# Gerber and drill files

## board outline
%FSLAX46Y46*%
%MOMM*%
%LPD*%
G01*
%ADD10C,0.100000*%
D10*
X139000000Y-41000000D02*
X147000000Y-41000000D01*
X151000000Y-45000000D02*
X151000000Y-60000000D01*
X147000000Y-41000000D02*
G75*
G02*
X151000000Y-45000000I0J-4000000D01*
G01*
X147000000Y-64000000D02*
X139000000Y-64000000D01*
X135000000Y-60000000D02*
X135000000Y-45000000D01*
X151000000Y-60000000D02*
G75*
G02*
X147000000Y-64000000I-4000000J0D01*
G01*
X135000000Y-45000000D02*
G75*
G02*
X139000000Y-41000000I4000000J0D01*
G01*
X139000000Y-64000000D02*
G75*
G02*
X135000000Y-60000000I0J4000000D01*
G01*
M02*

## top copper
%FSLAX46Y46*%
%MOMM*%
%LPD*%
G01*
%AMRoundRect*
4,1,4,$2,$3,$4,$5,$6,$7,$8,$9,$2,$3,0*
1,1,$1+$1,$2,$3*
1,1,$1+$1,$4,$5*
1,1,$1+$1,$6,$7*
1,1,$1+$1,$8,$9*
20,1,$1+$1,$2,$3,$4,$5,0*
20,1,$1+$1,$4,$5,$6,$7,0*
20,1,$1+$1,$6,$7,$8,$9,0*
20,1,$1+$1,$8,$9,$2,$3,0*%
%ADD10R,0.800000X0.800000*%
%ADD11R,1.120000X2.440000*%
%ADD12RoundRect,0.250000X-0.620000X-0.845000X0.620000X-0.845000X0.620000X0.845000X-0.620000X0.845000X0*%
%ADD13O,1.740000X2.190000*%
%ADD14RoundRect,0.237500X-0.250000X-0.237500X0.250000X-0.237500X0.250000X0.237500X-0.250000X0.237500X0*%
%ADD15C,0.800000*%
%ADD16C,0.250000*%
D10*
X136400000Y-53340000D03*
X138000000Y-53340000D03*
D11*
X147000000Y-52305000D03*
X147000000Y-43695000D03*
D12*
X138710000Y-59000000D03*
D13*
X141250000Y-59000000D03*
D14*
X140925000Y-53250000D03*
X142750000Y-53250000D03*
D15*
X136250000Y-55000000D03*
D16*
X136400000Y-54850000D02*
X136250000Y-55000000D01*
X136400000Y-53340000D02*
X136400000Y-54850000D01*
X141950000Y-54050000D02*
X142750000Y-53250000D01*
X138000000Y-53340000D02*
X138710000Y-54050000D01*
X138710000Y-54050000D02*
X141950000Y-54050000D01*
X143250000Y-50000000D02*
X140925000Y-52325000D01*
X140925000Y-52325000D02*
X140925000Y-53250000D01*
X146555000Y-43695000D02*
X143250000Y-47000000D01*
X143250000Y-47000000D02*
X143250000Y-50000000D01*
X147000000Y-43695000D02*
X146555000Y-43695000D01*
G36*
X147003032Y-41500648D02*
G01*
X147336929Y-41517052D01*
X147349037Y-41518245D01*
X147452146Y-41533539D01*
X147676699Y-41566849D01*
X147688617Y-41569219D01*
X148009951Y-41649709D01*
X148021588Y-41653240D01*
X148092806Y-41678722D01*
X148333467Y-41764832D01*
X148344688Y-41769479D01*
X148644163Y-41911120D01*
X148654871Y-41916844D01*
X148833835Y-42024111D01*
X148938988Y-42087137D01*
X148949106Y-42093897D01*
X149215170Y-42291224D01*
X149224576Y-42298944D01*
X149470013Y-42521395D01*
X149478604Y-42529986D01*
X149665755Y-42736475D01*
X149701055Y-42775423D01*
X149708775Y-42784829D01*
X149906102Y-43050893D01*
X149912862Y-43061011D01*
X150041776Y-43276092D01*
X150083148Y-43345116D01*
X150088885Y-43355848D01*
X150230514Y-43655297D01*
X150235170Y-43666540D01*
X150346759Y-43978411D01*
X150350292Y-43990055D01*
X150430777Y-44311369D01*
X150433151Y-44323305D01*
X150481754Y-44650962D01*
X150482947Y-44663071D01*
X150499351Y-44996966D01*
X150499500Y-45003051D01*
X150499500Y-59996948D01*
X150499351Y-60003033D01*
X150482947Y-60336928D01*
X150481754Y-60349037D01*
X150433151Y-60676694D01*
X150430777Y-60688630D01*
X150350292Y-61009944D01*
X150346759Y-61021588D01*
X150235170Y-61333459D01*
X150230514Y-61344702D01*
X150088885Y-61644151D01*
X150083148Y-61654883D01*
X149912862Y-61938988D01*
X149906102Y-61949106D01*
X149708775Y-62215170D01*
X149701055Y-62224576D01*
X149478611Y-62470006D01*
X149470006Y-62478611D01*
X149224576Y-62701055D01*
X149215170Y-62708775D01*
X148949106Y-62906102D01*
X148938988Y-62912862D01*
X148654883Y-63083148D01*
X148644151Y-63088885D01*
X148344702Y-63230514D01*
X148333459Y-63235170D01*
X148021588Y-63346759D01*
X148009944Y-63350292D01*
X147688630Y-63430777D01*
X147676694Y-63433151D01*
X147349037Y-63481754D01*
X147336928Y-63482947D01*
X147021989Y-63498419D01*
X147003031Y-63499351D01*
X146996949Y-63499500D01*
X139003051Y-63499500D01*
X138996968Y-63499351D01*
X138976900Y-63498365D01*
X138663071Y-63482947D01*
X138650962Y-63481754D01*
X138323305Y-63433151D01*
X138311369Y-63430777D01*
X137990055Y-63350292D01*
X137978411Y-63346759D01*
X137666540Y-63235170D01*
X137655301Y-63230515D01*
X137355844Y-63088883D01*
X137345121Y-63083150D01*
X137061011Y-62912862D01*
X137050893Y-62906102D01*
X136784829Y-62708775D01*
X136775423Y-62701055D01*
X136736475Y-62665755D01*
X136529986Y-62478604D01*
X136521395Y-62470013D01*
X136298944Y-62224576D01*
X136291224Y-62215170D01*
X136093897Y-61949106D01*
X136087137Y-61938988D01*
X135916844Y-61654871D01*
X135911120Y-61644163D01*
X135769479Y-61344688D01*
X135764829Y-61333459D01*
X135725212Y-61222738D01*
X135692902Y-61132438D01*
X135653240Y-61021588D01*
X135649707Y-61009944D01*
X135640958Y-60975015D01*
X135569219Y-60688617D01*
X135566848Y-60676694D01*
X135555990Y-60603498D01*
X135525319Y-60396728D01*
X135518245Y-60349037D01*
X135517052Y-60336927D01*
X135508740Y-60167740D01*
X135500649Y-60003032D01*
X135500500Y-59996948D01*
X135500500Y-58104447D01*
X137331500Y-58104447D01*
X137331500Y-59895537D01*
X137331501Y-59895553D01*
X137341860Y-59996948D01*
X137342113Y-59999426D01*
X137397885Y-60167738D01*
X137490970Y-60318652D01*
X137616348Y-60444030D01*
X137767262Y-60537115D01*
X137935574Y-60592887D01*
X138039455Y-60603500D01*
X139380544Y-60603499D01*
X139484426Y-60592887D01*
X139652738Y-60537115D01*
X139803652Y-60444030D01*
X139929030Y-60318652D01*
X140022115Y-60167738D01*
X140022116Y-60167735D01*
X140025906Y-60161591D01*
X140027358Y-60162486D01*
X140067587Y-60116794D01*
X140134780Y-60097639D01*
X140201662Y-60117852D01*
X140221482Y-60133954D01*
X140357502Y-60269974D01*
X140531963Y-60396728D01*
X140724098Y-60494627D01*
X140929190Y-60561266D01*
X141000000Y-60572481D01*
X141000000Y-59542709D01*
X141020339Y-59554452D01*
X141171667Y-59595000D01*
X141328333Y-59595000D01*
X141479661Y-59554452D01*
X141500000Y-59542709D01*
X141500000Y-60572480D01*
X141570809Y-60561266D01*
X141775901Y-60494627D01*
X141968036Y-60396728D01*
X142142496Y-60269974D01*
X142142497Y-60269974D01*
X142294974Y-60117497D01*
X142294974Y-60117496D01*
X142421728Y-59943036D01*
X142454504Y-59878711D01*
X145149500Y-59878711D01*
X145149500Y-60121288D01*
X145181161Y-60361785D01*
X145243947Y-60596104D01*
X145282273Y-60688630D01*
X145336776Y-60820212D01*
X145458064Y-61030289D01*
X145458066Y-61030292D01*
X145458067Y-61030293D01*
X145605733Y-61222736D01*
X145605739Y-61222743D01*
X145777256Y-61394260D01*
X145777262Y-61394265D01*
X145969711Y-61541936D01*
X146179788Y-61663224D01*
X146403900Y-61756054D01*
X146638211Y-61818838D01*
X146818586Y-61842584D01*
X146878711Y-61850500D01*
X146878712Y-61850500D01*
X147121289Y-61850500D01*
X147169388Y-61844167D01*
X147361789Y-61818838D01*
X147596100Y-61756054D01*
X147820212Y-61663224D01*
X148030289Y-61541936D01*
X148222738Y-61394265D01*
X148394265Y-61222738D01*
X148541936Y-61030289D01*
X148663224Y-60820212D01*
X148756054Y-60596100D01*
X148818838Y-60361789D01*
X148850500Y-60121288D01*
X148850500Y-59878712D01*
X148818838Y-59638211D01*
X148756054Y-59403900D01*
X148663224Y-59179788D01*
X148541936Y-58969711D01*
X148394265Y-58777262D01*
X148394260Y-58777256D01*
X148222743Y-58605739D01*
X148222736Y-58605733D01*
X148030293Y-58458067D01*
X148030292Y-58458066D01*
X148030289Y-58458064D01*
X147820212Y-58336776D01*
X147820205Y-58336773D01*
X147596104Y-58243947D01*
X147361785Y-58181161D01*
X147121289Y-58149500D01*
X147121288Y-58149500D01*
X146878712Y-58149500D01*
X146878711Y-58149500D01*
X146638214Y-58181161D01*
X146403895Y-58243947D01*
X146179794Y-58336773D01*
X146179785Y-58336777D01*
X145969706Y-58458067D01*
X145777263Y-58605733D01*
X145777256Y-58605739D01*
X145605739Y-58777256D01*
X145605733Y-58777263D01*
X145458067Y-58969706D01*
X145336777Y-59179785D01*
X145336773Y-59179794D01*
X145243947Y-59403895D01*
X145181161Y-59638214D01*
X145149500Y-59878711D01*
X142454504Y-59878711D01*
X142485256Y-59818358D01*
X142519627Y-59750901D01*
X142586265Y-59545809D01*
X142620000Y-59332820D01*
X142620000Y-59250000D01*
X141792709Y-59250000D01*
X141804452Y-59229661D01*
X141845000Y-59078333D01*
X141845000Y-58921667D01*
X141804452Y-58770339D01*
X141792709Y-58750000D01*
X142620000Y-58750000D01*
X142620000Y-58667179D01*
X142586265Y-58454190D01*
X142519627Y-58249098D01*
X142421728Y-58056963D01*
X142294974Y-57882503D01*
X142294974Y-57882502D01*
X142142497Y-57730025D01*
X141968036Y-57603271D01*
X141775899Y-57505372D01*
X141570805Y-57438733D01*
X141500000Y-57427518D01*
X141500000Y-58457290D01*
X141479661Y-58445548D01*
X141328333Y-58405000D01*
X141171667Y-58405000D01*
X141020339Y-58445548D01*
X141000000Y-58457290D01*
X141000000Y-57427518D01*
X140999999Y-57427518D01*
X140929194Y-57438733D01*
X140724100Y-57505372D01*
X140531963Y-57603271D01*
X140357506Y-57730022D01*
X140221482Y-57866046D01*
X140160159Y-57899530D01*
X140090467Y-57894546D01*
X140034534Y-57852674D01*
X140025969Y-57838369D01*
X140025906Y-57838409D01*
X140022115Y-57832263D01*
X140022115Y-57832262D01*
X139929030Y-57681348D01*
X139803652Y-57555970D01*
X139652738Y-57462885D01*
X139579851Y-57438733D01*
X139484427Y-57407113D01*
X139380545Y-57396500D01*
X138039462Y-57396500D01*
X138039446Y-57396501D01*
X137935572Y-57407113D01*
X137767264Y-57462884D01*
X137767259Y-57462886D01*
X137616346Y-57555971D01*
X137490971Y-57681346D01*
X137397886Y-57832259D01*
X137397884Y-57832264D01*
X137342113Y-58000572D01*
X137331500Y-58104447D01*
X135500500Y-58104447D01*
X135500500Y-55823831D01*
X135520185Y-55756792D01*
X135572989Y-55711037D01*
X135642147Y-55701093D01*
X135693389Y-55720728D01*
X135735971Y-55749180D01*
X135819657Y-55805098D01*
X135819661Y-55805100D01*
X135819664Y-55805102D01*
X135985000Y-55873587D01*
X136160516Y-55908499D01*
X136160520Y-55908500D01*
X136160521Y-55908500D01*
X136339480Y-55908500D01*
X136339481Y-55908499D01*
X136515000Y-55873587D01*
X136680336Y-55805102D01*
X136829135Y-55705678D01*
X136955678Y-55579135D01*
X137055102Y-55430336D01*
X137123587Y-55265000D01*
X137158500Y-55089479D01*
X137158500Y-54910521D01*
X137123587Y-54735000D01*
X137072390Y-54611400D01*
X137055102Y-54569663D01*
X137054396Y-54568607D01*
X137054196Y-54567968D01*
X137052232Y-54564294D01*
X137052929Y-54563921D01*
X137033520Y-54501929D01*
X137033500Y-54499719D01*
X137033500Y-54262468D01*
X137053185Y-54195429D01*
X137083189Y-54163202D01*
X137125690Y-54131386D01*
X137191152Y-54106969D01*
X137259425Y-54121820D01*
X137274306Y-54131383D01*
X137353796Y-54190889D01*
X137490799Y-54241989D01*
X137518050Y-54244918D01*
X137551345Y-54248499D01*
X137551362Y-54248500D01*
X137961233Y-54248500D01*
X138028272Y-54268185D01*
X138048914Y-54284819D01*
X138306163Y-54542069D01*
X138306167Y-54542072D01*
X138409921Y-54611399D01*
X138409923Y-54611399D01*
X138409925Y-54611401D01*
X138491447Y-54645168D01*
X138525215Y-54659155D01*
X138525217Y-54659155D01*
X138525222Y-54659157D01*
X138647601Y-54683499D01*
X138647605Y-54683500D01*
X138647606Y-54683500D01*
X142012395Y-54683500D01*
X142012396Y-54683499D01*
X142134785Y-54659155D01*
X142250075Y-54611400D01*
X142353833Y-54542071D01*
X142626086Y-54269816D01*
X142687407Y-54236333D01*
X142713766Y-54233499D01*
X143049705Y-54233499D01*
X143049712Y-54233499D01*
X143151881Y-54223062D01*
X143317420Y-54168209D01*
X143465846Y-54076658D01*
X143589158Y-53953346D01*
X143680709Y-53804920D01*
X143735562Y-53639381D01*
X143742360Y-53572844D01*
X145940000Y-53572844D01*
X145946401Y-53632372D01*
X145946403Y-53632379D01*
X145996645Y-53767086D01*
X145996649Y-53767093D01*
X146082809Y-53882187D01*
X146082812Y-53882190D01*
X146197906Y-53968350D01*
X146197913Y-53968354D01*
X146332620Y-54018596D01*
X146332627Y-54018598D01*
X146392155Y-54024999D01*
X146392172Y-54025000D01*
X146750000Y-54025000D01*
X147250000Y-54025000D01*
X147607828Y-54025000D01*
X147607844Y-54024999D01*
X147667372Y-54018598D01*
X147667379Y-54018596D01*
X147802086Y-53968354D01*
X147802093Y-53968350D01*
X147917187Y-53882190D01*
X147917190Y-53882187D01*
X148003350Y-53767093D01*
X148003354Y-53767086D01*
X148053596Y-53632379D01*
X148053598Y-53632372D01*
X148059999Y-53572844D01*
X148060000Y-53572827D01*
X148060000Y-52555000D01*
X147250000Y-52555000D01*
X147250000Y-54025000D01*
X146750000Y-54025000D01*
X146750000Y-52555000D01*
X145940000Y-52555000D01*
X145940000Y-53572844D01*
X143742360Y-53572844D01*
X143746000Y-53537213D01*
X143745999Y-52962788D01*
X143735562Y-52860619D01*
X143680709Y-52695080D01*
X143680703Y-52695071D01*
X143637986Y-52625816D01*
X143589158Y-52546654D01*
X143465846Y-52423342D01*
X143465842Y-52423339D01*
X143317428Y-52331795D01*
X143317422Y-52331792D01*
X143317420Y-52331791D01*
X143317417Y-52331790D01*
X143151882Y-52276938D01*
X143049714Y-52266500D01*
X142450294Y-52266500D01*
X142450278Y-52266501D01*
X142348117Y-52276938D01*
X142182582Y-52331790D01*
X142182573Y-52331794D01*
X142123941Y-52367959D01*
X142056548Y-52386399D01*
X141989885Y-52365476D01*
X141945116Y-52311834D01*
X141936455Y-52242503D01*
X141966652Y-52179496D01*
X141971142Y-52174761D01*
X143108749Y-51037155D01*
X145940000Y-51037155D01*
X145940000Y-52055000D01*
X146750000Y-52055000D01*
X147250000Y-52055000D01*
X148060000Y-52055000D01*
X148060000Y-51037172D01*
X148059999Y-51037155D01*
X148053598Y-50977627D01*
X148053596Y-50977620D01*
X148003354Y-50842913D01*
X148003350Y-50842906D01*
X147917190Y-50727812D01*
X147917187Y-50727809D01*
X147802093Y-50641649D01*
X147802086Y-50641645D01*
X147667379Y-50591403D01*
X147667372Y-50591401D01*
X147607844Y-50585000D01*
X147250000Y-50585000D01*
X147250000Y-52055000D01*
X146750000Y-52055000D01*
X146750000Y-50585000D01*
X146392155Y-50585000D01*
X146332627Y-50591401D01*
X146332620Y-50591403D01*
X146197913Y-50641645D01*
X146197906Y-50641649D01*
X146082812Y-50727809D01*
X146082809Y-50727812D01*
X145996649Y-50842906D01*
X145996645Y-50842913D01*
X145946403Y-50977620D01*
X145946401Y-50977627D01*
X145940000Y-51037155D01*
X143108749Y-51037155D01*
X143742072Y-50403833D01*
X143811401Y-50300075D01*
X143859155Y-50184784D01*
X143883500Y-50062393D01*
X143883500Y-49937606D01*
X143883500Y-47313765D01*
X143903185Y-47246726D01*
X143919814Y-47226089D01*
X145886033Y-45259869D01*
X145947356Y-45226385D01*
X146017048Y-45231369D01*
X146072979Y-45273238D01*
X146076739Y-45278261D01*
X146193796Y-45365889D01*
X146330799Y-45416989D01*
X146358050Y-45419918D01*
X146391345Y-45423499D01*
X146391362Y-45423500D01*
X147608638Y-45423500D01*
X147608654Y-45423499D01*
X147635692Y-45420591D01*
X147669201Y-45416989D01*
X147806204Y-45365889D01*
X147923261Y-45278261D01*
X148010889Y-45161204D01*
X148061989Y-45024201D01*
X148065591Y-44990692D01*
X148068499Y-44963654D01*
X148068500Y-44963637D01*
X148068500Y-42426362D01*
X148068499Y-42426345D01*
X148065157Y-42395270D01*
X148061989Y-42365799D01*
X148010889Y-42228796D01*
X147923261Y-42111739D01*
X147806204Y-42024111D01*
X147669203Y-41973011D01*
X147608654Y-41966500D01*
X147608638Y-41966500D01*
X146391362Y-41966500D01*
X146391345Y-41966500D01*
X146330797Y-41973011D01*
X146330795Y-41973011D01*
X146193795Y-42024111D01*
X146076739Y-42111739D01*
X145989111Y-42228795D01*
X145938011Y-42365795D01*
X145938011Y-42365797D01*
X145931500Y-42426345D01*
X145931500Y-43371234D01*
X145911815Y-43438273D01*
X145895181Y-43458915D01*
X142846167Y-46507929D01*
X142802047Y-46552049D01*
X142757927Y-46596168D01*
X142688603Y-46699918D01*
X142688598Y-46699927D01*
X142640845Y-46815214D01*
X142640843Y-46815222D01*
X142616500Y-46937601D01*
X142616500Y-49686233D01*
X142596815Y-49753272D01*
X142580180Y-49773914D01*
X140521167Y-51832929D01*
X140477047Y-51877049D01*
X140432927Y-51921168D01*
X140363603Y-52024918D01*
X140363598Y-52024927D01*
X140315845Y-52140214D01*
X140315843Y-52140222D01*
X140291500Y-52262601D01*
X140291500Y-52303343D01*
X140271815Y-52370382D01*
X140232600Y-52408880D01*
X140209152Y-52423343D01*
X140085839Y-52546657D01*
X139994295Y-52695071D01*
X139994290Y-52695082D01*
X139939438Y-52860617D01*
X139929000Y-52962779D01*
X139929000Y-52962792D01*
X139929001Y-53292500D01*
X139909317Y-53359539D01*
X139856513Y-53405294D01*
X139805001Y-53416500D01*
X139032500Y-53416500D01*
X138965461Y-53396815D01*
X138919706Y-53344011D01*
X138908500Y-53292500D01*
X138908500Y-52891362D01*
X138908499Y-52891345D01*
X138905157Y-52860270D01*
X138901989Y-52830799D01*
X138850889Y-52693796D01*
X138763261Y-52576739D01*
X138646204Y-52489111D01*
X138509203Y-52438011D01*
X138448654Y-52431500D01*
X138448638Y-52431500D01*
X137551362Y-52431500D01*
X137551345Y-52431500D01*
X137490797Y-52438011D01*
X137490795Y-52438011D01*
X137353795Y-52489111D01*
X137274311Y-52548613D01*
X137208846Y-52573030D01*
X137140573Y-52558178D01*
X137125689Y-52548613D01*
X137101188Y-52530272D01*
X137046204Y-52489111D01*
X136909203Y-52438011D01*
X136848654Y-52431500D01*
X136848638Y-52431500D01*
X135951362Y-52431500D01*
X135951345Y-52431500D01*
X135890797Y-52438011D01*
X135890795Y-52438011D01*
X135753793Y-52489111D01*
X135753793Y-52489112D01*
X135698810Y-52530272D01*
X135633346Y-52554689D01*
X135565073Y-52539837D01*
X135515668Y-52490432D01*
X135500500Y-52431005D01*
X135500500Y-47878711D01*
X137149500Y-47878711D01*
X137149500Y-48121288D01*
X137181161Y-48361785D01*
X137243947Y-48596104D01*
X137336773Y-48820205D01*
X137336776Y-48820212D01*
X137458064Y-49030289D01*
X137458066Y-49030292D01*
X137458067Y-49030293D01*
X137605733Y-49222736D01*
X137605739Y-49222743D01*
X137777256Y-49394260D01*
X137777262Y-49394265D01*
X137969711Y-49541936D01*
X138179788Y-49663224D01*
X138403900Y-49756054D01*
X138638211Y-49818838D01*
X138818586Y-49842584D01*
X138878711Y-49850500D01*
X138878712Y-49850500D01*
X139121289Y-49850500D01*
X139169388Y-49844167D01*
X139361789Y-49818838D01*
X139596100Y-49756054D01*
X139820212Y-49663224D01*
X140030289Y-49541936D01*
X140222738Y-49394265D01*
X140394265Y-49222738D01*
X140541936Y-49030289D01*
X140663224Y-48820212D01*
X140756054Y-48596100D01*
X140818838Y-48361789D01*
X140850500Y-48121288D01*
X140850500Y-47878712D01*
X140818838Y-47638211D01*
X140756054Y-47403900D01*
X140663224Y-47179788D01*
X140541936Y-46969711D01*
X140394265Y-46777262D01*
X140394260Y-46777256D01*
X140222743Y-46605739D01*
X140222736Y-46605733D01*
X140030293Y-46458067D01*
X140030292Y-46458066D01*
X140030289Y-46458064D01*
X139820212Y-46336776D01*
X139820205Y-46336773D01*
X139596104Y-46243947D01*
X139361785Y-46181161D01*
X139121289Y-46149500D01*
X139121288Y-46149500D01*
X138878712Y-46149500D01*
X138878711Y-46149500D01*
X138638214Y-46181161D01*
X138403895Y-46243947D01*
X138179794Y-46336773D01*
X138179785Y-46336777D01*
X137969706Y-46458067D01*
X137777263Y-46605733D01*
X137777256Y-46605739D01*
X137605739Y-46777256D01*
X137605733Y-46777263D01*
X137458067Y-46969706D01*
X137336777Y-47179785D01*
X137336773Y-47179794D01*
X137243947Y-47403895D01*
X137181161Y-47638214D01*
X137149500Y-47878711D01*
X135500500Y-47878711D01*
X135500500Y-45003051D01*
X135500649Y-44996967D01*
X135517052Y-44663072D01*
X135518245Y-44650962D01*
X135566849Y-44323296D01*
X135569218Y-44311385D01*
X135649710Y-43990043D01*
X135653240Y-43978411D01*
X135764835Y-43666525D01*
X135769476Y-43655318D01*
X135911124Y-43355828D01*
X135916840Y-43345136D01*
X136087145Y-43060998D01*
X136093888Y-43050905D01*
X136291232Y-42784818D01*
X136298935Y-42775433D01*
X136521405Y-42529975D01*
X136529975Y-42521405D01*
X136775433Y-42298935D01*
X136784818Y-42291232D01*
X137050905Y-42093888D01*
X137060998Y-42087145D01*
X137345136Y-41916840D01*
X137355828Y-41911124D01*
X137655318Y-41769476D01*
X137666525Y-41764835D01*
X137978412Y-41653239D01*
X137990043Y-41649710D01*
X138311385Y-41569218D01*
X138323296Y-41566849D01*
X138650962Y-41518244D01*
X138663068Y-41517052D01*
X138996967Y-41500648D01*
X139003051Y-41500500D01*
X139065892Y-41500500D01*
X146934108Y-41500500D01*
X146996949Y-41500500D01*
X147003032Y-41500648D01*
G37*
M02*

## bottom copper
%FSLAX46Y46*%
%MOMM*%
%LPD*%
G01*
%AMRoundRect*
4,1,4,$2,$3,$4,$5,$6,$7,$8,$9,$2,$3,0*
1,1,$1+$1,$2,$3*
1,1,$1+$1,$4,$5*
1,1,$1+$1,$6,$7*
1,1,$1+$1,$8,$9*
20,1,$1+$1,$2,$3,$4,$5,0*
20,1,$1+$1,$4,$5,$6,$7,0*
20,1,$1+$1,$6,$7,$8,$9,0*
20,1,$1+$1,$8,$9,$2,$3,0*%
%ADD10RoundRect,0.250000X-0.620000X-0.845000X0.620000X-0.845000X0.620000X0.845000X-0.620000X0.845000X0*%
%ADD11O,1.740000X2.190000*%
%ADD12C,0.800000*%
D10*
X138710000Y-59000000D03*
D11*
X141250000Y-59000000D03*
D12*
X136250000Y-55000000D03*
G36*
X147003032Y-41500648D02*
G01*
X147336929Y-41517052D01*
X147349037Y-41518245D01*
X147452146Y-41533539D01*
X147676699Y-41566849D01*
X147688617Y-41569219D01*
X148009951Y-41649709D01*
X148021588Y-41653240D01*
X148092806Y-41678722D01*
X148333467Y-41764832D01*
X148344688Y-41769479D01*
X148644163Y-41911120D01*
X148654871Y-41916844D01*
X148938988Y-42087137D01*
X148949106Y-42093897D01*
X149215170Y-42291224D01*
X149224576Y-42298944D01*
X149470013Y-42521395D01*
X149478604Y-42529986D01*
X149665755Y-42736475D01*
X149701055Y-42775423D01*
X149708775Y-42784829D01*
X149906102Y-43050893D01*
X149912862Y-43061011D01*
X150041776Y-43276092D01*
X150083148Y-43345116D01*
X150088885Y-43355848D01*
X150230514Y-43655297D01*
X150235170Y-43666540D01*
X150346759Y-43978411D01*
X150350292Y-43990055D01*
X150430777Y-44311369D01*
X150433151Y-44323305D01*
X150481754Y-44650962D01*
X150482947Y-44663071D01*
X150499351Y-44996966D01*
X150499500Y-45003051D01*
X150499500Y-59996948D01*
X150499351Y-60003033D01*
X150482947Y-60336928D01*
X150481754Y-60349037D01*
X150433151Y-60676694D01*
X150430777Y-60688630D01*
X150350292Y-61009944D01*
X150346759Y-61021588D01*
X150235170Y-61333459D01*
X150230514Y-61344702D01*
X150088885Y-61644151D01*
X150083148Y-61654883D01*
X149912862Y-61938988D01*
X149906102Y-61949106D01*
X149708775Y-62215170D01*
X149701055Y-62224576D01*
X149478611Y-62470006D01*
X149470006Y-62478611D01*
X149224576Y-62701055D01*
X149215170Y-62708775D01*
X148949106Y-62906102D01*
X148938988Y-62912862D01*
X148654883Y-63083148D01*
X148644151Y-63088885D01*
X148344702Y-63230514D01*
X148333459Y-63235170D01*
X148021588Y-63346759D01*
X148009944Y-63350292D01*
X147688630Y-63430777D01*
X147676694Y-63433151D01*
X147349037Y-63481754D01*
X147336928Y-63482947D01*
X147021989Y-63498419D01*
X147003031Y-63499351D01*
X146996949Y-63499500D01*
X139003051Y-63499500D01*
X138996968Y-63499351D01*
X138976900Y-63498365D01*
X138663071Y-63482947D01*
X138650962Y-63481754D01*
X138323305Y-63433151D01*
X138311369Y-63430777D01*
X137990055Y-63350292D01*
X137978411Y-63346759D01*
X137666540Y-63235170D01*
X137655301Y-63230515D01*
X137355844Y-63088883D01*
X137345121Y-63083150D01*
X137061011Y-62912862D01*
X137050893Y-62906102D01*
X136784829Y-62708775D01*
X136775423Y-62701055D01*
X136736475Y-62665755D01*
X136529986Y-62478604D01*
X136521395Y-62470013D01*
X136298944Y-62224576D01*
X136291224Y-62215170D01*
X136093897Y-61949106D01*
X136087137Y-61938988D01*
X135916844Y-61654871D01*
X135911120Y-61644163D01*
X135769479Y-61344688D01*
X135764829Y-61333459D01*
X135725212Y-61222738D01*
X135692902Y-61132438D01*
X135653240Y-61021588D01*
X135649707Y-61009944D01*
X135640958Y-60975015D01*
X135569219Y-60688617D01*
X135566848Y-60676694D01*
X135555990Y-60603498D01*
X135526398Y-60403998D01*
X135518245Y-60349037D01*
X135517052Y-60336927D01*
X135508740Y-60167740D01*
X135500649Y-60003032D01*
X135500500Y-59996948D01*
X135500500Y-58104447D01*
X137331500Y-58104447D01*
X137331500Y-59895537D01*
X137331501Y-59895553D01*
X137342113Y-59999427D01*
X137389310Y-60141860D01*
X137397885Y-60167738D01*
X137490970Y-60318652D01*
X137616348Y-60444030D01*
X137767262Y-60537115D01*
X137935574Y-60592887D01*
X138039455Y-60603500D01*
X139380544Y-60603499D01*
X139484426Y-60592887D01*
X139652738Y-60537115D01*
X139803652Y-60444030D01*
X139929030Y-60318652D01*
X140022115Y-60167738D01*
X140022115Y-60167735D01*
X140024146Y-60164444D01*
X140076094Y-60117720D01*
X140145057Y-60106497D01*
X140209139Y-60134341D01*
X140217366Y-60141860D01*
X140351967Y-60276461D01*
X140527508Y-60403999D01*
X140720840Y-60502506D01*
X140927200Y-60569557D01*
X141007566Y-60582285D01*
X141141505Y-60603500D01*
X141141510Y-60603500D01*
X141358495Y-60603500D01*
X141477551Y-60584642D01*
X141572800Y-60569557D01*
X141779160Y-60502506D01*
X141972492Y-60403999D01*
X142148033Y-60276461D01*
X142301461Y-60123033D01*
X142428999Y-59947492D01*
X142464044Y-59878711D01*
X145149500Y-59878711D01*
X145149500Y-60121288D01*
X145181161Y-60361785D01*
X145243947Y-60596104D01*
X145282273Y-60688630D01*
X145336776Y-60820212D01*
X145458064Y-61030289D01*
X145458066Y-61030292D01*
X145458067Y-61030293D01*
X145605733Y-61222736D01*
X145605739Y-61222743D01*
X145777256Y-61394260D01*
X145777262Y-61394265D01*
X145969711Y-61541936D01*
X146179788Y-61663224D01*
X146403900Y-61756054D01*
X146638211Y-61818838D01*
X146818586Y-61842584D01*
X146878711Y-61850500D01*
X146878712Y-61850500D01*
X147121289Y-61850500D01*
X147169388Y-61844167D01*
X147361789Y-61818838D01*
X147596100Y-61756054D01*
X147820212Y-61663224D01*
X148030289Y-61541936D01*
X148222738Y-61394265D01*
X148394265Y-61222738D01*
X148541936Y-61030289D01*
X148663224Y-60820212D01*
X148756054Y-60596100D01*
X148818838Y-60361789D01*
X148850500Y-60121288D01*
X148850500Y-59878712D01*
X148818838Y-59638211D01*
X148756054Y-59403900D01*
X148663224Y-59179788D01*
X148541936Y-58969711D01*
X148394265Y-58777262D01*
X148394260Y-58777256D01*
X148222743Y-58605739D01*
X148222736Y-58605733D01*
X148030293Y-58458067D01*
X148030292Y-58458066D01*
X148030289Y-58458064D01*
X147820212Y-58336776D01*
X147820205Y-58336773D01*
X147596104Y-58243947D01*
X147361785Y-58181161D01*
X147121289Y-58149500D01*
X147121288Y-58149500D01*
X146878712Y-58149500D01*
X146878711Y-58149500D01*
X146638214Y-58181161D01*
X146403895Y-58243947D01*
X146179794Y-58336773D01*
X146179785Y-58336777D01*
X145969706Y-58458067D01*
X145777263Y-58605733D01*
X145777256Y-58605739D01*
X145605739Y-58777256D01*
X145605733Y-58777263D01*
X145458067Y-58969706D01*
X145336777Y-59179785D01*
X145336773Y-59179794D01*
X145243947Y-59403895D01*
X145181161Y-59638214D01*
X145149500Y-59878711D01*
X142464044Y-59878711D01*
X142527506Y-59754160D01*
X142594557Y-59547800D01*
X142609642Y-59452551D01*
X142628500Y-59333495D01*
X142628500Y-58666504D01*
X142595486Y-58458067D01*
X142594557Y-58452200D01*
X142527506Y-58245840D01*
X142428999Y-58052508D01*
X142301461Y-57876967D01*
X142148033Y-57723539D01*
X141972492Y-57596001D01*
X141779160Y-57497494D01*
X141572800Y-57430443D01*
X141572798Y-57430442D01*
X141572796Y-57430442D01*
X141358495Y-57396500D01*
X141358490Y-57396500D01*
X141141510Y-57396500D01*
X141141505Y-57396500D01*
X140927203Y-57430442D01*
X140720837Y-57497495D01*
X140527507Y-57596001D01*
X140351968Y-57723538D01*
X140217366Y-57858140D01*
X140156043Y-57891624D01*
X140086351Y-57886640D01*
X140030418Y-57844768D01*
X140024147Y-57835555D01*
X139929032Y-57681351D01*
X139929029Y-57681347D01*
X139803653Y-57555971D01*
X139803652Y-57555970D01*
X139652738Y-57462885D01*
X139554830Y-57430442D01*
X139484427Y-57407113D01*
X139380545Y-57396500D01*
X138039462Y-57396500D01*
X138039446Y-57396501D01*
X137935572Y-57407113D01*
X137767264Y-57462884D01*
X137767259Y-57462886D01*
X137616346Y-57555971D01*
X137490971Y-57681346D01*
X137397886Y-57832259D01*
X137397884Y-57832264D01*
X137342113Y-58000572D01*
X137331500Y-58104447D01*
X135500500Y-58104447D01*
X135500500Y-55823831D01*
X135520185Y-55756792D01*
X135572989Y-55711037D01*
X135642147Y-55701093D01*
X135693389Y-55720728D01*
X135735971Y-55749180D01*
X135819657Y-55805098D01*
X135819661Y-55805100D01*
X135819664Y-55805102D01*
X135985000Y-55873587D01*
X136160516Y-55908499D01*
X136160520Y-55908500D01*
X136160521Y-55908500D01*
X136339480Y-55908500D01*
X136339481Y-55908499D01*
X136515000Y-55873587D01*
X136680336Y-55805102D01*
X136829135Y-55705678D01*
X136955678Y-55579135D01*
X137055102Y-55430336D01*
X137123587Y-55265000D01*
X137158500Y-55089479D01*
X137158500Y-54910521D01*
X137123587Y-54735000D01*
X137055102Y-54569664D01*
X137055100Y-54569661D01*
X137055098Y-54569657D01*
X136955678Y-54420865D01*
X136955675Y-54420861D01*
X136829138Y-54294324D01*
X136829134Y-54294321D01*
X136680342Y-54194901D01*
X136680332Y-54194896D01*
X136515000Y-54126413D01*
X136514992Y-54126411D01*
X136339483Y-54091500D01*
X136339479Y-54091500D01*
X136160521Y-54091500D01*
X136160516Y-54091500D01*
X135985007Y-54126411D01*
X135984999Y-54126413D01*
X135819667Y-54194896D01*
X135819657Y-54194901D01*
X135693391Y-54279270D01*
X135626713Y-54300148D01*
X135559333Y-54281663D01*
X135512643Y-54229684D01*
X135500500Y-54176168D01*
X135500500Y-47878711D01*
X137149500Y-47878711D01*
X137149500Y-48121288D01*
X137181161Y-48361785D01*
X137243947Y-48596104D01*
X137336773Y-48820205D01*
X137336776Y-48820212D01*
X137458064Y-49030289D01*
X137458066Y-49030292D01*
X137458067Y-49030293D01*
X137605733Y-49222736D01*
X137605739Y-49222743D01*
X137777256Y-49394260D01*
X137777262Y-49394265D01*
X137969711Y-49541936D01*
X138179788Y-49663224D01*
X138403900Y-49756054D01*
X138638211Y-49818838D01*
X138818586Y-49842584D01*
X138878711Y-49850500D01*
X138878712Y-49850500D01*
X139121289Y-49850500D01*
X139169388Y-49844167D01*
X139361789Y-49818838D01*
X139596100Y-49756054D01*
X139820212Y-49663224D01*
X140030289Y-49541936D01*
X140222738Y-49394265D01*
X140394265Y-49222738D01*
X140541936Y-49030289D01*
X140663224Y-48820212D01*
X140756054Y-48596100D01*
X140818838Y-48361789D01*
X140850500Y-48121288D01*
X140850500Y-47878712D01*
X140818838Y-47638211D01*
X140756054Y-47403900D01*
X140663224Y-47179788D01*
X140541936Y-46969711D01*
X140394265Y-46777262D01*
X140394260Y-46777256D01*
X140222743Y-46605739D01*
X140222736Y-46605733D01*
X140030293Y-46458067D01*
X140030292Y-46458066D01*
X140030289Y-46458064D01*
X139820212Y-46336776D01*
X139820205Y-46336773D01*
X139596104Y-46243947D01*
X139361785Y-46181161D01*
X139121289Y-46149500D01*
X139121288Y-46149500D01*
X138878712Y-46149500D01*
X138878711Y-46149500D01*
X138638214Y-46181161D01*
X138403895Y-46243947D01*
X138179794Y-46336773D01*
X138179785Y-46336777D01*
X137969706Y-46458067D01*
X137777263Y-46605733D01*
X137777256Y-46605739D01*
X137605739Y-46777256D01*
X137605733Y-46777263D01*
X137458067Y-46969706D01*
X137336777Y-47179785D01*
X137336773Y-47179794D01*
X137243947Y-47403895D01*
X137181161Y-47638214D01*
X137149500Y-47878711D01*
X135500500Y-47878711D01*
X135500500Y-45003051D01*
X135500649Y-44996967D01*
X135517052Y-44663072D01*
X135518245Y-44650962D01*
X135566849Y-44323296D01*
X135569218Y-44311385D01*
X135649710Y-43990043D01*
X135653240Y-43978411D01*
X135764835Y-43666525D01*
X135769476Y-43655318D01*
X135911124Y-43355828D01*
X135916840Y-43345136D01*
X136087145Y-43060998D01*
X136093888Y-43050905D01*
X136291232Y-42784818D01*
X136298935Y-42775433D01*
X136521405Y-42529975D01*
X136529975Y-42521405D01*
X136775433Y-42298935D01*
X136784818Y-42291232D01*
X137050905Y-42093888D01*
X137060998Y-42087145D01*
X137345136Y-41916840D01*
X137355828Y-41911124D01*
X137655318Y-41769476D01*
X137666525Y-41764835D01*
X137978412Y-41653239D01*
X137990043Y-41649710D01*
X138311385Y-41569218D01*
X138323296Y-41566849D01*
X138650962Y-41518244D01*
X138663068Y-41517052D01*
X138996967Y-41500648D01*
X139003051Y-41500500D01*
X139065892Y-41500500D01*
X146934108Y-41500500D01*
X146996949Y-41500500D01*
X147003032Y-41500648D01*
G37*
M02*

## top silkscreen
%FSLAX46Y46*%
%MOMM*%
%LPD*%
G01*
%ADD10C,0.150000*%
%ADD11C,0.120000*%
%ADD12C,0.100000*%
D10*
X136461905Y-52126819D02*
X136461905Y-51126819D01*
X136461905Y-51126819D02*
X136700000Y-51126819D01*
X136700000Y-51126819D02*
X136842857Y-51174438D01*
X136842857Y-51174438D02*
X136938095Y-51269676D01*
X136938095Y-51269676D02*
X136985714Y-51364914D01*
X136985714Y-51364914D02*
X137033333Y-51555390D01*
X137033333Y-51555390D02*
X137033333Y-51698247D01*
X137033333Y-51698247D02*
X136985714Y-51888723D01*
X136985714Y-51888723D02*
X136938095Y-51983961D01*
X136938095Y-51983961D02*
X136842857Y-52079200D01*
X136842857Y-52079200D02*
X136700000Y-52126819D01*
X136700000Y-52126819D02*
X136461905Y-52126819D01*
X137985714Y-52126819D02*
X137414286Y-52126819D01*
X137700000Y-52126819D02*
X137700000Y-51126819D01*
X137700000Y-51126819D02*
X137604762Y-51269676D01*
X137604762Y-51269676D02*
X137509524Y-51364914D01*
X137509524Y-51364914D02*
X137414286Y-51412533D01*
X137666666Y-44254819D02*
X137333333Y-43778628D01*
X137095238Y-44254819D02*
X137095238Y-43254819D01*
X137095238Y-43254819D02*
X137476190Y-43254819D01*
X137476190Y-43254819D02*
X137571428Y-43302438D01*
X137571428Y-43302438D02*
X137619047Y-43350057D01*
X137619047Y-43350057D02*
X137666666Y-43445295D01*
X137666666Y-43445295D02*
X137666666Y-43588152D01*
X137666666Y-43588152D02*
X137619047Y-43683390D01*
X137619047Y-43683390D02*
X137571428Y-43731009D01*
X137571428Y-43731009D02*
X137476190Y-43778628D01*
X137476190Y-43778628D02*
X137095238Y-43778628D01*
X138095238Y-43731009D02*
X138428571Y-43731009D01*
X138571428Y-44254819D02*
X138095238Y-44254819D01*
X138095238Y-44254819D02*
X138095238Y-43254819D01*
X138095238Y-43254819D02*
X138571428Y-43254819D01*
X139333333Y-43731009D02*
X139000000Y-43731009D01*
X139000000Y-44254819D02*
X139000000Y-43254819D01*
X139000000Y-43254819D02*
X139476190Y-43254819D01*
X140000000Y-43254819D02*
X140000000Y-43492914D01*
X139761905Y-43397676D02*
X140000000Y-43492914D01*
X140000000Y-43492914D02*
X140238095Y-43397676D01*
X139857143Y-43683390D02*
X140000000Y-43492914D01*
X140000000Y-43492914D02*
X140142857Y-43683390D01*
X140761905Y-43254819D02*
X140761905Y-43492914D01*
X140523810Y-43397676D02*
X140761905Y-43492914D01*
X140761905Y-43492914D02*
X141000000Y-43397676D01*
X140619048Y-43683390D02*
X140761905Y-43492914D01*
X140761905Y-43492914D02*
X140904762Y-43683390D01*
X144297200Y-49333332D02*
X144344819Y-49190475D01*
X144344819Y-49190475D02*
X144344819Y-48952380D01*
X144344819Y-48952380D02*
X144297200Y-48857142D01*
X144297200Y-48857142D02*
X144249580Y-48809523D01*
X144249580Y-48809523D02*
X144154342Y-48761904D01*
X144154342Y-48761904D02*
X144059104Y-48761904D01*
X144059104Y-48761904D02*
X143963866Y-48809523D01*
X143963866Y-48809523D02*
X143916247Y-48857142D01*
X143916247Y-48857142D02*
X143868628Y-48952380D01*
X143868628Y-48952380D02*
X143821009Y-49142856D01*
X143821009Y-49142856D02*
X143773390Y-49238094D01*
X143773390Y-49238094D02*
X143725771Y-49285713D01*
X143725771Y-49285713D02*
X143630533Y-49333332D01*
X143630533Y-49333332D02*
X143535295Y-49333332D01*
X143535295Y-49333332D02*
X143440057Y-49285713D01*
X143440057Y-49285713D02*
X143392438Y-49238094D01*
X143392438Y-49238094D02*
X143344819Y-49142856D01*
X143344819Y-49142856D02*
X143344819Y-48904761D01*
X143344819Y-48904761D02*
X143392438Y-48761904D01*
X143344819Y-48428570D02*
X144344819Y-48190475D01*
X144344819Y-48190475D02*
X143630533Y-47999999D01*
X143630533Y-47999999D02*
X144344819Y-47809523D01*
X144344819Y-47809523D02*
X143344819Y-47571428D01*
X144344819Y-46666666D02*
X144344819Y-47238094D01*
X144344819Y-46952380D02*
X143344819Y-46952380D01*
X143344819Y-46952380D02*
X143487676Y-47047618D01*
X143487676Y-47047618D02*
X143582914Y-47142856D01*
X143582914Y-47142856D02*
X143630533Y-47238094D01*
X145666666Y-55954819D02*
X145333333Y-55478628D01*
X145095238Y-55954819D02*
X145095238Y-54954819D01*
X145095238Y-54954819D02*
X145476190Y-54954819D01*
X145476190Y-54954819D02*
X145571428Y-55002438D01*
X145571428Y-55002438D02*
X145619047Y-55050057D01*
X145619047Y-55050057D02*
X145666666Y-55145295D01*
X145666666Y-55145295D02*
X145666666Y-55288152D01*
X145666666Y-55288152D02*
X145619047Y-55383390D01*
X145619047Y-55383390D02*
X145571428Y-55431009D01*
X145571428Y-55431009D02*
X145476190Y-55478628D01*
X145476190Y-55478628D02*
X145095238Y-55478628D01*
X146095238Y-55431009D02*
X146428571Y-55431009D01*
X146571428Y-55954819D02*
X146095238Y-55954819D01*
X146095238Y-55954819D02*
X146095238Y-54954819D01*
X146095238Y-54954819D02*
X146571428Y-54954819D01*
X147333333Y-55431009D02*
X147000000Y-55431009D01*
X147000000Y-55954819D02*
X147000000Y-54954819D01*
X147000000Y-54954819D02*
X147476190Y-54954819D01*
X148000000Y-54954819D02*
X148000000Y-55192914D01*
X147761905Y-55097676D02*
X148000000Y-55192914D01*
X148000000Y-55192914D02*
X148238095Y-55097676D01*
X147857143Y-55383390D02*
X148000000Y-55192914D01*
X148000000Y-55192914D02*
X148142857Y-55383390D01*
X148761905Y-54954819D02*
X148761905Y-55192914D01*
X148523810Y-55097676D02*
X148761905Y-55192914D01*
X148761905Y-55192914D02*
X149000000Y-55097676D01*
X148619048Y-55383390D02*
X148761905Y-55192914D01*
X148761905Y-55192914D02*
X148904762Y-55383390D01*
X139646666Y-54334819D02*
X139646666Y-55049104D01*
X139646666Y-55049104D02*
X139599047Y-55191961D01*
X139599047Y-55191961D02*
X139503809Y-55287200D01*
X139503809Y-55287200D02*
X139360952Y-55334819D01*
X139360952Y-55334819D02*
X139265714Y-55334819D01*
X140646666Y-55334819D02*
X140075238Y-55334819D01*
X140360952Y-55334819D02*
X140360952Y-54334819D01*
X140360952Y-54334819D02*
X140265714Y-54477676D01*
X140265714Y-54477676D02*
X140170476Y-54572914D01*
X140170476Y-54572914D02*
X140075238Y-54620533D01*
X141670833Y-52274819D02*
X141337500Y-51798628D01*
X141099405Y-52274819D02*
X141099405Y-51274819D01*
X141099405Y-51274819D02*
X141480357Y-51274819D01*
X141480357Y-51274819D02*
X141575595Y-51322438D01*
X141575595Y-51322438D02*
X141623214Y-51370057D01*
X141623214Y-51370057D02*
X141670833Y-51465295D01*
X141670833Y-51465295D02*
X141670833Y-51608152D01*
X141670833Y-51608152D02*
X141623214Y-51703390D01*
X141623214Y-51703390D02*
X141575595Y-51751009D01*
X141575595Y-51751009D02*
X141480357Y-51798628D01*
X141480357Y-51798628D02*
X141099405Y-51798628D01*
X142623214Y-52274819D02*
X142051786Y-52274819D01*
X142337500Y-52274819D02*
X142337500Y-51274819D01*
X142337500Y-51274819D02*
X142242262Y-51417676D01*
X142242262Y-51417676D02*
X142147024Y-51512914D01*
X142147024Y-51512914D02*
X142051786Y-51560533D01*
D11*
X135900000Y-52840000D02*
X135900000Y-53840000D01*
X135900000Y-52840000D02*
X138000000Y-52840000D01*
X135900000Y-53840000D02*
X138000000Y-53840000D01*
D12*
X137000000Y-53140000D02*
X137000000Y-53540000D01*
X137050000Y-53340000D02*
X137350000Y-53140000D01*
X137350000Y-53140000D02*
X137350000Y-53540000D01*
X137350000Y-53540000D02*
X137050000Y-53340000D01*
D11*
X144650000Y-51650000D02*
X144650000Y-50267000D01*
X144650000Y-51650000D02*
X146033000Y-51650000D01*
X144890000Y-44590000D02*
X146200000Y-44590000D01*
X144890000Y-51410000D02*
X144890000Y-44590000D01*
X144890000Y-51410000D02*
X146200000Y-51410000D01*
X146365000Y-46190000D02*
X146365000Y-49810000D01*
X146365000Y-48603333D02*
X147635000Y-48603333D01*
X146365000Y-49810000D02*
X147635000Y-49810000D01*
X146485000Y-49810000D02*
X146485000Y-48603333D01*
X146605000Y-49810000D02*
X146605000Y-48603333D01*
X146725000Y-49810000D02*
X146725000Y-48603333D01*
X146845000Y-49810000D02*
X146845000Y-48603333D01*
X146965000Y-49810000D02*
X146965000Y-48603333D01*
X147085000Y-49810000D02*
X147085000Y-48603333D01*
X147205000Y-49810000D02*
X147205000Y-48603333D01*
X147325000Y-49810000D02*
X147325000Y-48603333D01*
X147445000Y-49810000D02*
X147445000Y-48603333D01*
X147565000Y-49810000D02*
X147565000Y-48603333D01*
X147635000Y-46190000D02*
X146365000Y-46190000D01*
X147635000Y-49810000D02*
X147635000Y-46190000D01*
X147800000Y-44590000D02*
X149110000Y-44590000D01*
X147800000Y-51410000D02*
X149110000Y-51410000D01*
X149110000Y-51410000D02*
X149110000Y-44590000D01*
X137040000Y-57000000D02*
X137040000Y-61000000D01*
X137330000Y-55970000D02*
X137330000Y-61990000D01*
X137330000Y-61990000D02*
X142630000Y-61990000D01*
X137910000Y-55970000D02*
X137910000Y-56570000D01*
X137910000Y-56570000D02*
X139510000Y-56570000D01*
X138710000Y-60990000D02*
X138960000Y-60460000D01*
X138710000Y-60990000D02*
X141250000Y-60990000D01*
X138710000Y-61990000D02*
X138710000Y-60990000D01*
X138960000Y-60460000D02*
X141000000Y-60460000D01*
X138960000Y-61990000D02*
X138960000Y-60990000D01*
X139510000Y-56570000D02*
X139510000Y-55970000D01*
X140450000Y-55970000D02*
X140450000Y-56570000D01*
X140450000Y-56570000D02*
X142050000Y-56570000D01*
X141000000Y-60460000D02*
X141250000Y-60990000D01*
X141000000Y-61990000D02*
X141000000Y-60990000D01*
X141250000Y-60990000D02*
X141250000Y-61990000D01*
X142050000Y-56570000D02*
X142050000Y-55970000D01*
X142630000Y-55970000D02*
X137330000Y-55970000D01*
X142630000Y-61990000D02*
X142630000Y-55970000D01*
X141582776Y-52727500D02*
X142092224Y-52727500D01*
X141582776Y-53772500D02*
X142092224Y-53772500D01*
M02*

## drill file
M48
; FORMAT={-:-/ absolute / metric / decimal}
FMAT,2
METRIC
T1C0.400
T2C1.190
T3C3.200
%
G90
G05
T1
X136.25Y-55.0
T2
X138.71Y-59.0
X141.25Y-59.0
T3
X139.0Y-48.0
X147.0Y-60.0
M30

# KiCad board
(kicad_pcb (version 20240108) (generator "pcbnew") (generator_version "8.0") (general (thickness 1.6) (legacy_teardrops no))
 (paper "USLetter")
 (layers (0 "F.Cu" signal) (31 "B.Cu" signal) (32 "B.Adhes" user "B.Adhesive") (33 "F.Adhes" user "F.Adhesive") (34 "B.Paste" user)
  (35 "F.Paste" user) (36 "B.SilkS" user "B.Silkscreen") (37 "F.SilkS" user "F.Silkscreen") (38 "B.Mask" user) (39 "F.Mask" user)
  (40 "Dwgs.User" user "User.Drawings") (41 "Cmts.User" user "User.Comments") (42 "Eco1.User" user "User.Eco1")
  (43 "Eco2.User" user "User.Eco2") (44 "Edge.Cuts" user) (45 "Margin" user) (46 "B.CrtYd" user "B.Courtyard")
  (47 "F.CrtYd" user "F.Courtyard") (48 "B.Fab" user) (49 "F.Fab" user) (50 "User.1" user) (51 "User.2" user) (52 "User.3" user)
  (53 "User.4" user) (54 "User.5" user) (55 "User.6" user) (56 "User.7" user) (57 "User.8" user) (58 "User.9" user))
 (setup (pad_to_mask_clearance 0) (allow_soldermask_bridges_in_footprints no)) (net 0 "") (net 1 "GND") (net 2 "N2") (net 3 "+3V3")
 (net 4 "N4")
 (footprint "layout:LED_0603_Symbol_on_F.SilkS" (layer "F.Cu") (at 137.2 53.34)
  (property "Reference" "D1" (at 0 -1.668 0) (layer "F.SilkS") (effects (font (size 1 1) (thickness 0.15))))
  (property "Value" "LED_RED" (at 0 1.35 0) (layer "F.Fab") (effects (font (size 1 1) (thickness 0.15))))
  (fp_line (start -1.3 -0.5) (end -1.3 0.5) (stroke (width 0.12) (type solid)) (layer "F.SilkS"))
  (fp_line (start -1.3 -0.5) (end 0.8 -0.5) (stroke (width 0.12) (type solid)) (layer "F.SilkS"))
  (fp_line (start -1.3 0.5) (end 0.8 0.5) (stroke (width 0.12) (type solid)) (layer "F.SilkS"))
  (fp_line (start -0.2 -0.2) (end -0.2 0.2) (stroke (width 0.1) (type solid)) (layer "F.SilkS"))
  (fp_line (start -0.15 0) (end 0.15 -0.2) (stroke (width 0.1) (type solid)) (layer "F.SilkS"))
  (fp_line (start 0.15 -0.2) (end 0.15 0.2) (stroke (width 0.1) (type solid)) (layer "F.SilkS"))
  (fp_line (start 0.15 0.2) (end -0.15 0) (stroke (width 0.1) (type solid)) (layer "F.SilkS"))
  (pad "1" smd rect (at -0.8 0 180) (size 0.8 0.8) (layers "F.Cu" "F.Paste" "F.Mask") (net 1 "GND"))
  (pad "2" smd rect (at 0.8 0 180) (size 0.8 0.8) (layers "F.Cu" "F.Paste" "F.Mask") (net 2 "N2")))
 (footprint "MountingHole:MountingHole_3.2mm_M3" (layer "F.Cu") (at 139 48)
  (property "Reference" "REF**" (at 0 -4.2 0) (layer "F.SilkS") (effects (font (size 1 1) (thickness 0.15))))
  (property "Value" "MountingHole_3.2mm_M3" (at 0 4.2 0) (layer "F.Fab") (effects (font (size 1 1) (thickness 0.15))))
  (pad "" np_thru_hole circle (at 0 0) (size 3.2 3.2) (drill 3.2) (layers "*.Cu" "*.Mask")))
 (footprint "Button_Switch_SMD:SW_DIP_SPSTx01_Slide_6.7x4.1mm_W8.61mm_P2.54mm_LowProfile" (layer "F.Cu") (at 147 48 90)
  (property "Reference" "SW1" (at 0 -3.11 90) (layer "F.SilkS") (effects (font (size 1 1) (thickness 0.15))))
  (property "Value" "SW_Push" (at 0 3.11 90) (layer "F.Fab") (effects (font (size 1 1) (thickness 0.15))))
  (fp_line (start -3.65 -2.35) (end -2.267 -2.35) (stroke (width 0.12) (type solid)) (layer "F.SilkS"))
  (fp_line (start -3.65 -2.35) (end -3.65 -0.967) (stroke (width 0.12) (type solid)) (layer "F.SilkS"))
  (fp_line (start 3.41 -2.11) (end 3.41 -0.8) (stroke (width 0.12) (type solid)) (layer "F.SilkS"))
  (fp_line (start -3.41 -2.11) (end 3.41 -2.11) (stroke (width 0.12) (type solid)) (layer "F.SilkS"))
  (fp_line (start -3.41 -2.11) (end -3.41 -0.8) (stroke (width 0.12) (type solid)) (layer "F.SilkS"))
  (fp_line (start 1.81 -0.635) (end -1.81 -0.635) (stroke (width 0.12) (type solid)) (layer "F.SilkS"))
  (fp_line (start -0.603333 -0.635) (end -0.603333 0.635) (stroke (width 0.12) (type solid)) (layer "F.SilkS"))
  (fp_line (start -1.81 -0.635) (end -1.81 0.635) (stroke (width 0.12) (type solid)) (layer "F.SilkS"))
  (fp_line (start -1.81 -0.515) (end -0.603333 -0.515) (stroke (width 0.12) (type solid)) (layer "F.SilkS"))
  (fp_line (start -1.81 -0.395) (end -0.603333 -0.395) (stroke (width 0.12) (type solid)) (layer "F.SilkS"))
  (fp_line (start -1.81 -0.275) (end -0.603333 -0.275) (stroke (width 0.12) (type solid)) (layer "F.SilkS"))
  (fp_line (start -1.81 -0.155) (end -0.603333 -0.155) (stroke (width 0.12) (type solid)) (layer "F.SilkS"))
  (fp_line (start -1.81 -0.035) (end -0.603333 -0.035) (stroke (width 0.12) (type solid)) (layer "F.SilkS"))
  (fp_line (start -1.81 0.085) (end -0.603333 0.085) (stroke (width 0.12) (type solid)) (layer "F.SilkS"))
  (fp_line (start -1.81 0.205) (end -0.603333 0.205) (stroke (width 0.12) (type solid)) (layer "F.SilkS"))
  (fp_line (start -1.81 0.325) (end -0.603333 0.325) (stroke (width 0.12) (type solid)) (layer "F.SilkS"))
  (fp_line (start -1.81 0.445) (end -0.603333 0.445) (stroke (width 0.12) (type solid)) (layer "F.SilkS"))
  (fp_line (start -1.81 0.565) (end -0.603333 0.565) (stroke (width 0.12) (type solid)) (layer "F.SilkS"))
  (fp_line (start 1.81 0.635) (end 1.81 -0.635) (stroke (width 0.12) (type solid)) (layer "F.SilkS"))
  (fp_line (start -1.81 0.635) (end 1.81 0.635) (stroke (width 0.12) (type solid)) (layer "F.SilkS"))
  (fp_line (start 3.41 0.8) (end 3.41 2.11) (stroke (width 0.12) (type solid)) (layer "F.SilkS"))
  (fp_line (start -3.41 0.8) (end -3.41 2.11) (stroke (width 0.12) (type solid)) (layer "F.SilkS"))
  (fp_line (start -3.41 2.11) (end 3.41 2.11) (stroke (width 0.12) (type solid)) (layer "F.SilkS"))
  (pad "1" smd rect (at -4.305 0 90) (size 2.44 1.12) (layers "F.Cu" "F.Paste" "F.Mask") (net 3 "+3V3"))
  (pad "2" smd rect (at 4.305 0 90) (size 2.44 1.12) (layers "F.Cu" "F.Paste" "F.Mask") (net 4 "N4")))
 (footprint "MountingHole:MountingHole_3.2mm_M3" (layer "F.Cu") (at 147 60)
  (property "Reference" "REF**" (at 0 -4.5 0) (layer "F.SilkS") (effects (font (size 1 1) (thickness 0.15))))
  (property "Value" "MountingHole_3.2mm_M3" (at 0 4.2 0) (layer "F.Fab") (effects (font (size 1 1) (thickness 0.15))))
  (pad "" np_thru_hole circle (at 0 0) (size 3.2 3.2) (drill 3.2) (layers "*.Cu" "*.Mask")))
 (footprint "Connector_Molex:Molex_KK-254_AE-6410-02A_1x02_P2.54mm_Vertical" (layer "F.Cu") (at 138.71 59)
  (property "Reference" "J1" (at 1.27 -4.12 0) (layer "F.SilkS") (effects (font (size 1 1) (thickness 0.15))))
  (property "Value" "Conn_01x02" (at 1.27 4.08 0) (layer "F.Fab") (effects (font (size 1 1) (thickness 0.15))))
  (fp_line (start -1.67 -2) (end -1.67 2) (stroke (width 0.12) (type solid)) (layer "F.SilkS"))
  (fp_line (start -1.38 -3.03) (end -1.38 2.99) (stroke (width 0.12) (type solid)) (layer "F.SilkS"))
  (fp_line (start -1.38 2.99) (end 3.92 2.99) (stroke (width 0.12) (type solid)) (layer "F.SilkS"))
  (fp_line (start -0.8 -3.03) (end -0.8 -2.43) (stroke (width 0.12) (type solid)) (layer "F.SilkS"))
  (fp_line (start -0.8 -2.43) (end 0.8 -2.43) (stroke (width 0.12) (type solid)) (layer "F.SilkS"))
  (fp_line (start 0 1.99) (end 0.25 1.46) (stroke (width 0.12) (type solid)) (layer "F.SilkS"))
  (fp_line (start 0 1.99) (end 2.54 1.99) (stroke (width 0.12) (type solid)) (layer "F.SilkS"))
  (fp_line (start 0 2.99) (end 0 1.99) (stroke (width 0.12) (type solid)) (layer "F.SilkS"))
  (fp_line (start 0.25 1.46) (end 2.29 1.46) (stroke (width 0.12) (type solid)) (layer "F.SilkS"))
  (fp_line (start 0.25 2.99) (end 0.25 1.99) (stroke (width 0.12) (type solid)) (layer "F.SilkS"))
  (fp_line (start 0.8 -2.43) (end 0.8 -3.03) (stroke (width 0.12) (type solid)) (layer "F.SilkS"))
  (fp_line (start 1.74 -3.03) (end 1.74 -2.43) (stroke (width 0.12) (type solid)) (layer "F.SilkS"))
  (fp_line (start 1.74 -2.43) (end 3.34 -2.43) (stroke (width 0.12) (type solid)) (layer "F.SilkS"))
  (fp_line (start 2.29 1.46) (end 2.54 1.99) (stroke (width 0.12) (type solid)) (layer "F.SilkS"))
  (fp_line (start 2.29 2.99) (end 2.29 1.99) (stroke (width 0.12) (type solid)) (layer "F.SilkS"))
  (fp_line (start 2.54 1.99) (end 2.54 2.99) (stroke (width 0.12) (type solid)) (layer "F.SilkS"))
  (fp_line (start 3.34 -2.43) (end 3.34 -3.03) (stroke (width 0.12) (type solid)) (layer "F.SilkS"))
  (fp_line (start 3.92 -3.03) (end -1.38 -3.03) (stroke (width 0.12) (type solid)) (layer "F.SilkS"))
  (fp_line (start 3.92 2.99) (end 3.92 -3.03) (stroke (width 0.12) (type solid)) (layer "F.SilkS"))
  (pad "1" thru_hole roundrect (at 0 0) (size 1.74 2.19) (drill 1.19) (layers "*.Cu" "*.Mask") (remove_unused_layers no)
   (roundrect_rratio 0.143678) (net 1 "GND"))
  (pad "2" thru_hole oval (at 2.54 0) (size 1.74 2.19) (drill 1.19) (layers "*.Cu" "*.Mask") (remove_unused_layers no) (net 3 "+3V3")))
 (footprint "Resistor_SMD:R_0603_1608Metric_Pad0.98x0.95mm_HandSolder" (layer "F.Cu") (at 141.8375 53.25)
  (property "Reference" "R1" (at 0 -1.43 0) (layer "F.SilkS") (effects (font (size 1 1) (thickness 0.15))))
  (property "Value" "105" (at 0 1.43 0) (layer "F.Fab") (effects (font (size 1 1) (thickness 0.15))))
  (fp_line (start -0.254724 -0.5225) (end 0.254724 -0.5225) (stroke (width 0.12) (type solid)) (layer "F.SilkS"))
  (fp_line (start -0.254724 0.5225) (end 0.254724 0.5225) (stroke (width 0.12) (type solid)) (layer "F.SilkS"))
  (pad "1" smd roundrect (at -0.9125 0) (size 0.975 0.95) (layers "F.Cu" "F.Paste" "F.Mask") (roundrect_rratio 0.25) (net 4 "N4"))
  (pad "2" smd roundrect (at 0.9125 0) (size 0.975 0.95) (layers "F.Cu" "F.Paste" "F.Mask") (roundrect_rratio 0.25) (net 2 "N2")))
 (gr_line (start 139 41) (end 147 41) (stroke (width 0.1) (type default)) (layer "Edge.Cuts"))
 (gr_line (start 151 45) (end 151 60) (stroke (width 0.1) (type default)) (layer "Edge.Cuts"))
 (gr_arc (start 147 41) (mid 149.828427 42.171573) (end 151 45) (stroke (width 0.1) (type default)) (layer "Edge.Cuts"))
 (gr_line (start 147 64) (end 139 64) (stroke (width 0.1) (type default)) (layer "Edge.Cuts"))
 (gr_line (start 135 60) (end 135 45) (stroke (width 0.1) (type default)) (layer "Edge.Cuts"))
 (gr_arc (start 151 60) (mid 149.828427 62.828427) (end 147 64) (stroke (width 0.1) (type default)) (layer "Edge.Cuts"))
 (gr_arc (start 135 45) (mid 136.171573 42.171573) (end 139 41) (stroke (width 0.1) (type default)) (layer "Edge.Cuts"))
 (gr_arc (start 139 64) (mid 136.171573 62.828427) (end 135 60) (stroke (width 0.1) (type default)) (layer "Edge.Cuts"))
 (segment (start 136.4 54.85) (end 136.25 55) (width 0.25) (layer "F.Cu") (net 1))
 (segment (start 136.4 53.34) (end 136.4 54.85) (width 0.25) (layer "F.Cu") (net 1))
 (via (at 136.25 55) (size 0.8) (drill 0.4) (layers "F.Cu" "B.Cu") (free yes) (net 1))
 (segment (start 141.95 54.05) (end 142.75 53.25) (width 0.25) (layer "F.Cu") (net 2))
 (segment (start 138 53.34) (end 138.71 54.05) (width 0.25) (layer "F.Cu") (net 2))
 (segment (start 138.71 54.05) (end 141.95 54.05) (width 0.25) (layer "F.Cu") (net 2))
 (segment (start 143.25 50) (end 140.925 52.325) (width 0.25) (layer "F.Cu") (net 4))
 (segment (start 140.925 52.325) (end 140.925 53.25) (width 0.25) (layer "F.Cu") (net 4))
 (segment (start 146.555 43.695) (end 143.25 47) (width 0.25) (layer "F.Cu") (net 4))
 (segment (start 143.25 47) (end 143.25 50) (width 0.25) (layer "F.Cu") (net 4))
 (segment (start 147 43.695) (end 146.555 43.695) (width 0.25) (layer "F.Cu") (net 4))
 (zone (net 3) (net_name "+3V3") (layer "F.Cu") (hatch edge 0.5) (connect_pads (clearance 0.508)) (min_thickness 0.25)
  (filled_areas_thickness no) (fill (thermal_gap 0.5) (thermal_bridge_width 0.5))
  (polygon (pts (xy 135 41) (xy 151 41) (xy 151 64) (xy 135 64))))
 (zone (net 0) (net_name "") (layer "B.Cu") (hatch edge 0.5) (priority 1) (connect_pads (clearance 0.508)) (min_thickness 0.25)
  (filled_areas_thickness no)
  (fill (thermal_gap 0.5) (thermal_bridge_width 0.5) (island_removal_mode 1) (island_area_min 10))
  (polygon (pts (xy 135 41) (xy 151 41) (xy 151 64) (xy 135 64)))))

